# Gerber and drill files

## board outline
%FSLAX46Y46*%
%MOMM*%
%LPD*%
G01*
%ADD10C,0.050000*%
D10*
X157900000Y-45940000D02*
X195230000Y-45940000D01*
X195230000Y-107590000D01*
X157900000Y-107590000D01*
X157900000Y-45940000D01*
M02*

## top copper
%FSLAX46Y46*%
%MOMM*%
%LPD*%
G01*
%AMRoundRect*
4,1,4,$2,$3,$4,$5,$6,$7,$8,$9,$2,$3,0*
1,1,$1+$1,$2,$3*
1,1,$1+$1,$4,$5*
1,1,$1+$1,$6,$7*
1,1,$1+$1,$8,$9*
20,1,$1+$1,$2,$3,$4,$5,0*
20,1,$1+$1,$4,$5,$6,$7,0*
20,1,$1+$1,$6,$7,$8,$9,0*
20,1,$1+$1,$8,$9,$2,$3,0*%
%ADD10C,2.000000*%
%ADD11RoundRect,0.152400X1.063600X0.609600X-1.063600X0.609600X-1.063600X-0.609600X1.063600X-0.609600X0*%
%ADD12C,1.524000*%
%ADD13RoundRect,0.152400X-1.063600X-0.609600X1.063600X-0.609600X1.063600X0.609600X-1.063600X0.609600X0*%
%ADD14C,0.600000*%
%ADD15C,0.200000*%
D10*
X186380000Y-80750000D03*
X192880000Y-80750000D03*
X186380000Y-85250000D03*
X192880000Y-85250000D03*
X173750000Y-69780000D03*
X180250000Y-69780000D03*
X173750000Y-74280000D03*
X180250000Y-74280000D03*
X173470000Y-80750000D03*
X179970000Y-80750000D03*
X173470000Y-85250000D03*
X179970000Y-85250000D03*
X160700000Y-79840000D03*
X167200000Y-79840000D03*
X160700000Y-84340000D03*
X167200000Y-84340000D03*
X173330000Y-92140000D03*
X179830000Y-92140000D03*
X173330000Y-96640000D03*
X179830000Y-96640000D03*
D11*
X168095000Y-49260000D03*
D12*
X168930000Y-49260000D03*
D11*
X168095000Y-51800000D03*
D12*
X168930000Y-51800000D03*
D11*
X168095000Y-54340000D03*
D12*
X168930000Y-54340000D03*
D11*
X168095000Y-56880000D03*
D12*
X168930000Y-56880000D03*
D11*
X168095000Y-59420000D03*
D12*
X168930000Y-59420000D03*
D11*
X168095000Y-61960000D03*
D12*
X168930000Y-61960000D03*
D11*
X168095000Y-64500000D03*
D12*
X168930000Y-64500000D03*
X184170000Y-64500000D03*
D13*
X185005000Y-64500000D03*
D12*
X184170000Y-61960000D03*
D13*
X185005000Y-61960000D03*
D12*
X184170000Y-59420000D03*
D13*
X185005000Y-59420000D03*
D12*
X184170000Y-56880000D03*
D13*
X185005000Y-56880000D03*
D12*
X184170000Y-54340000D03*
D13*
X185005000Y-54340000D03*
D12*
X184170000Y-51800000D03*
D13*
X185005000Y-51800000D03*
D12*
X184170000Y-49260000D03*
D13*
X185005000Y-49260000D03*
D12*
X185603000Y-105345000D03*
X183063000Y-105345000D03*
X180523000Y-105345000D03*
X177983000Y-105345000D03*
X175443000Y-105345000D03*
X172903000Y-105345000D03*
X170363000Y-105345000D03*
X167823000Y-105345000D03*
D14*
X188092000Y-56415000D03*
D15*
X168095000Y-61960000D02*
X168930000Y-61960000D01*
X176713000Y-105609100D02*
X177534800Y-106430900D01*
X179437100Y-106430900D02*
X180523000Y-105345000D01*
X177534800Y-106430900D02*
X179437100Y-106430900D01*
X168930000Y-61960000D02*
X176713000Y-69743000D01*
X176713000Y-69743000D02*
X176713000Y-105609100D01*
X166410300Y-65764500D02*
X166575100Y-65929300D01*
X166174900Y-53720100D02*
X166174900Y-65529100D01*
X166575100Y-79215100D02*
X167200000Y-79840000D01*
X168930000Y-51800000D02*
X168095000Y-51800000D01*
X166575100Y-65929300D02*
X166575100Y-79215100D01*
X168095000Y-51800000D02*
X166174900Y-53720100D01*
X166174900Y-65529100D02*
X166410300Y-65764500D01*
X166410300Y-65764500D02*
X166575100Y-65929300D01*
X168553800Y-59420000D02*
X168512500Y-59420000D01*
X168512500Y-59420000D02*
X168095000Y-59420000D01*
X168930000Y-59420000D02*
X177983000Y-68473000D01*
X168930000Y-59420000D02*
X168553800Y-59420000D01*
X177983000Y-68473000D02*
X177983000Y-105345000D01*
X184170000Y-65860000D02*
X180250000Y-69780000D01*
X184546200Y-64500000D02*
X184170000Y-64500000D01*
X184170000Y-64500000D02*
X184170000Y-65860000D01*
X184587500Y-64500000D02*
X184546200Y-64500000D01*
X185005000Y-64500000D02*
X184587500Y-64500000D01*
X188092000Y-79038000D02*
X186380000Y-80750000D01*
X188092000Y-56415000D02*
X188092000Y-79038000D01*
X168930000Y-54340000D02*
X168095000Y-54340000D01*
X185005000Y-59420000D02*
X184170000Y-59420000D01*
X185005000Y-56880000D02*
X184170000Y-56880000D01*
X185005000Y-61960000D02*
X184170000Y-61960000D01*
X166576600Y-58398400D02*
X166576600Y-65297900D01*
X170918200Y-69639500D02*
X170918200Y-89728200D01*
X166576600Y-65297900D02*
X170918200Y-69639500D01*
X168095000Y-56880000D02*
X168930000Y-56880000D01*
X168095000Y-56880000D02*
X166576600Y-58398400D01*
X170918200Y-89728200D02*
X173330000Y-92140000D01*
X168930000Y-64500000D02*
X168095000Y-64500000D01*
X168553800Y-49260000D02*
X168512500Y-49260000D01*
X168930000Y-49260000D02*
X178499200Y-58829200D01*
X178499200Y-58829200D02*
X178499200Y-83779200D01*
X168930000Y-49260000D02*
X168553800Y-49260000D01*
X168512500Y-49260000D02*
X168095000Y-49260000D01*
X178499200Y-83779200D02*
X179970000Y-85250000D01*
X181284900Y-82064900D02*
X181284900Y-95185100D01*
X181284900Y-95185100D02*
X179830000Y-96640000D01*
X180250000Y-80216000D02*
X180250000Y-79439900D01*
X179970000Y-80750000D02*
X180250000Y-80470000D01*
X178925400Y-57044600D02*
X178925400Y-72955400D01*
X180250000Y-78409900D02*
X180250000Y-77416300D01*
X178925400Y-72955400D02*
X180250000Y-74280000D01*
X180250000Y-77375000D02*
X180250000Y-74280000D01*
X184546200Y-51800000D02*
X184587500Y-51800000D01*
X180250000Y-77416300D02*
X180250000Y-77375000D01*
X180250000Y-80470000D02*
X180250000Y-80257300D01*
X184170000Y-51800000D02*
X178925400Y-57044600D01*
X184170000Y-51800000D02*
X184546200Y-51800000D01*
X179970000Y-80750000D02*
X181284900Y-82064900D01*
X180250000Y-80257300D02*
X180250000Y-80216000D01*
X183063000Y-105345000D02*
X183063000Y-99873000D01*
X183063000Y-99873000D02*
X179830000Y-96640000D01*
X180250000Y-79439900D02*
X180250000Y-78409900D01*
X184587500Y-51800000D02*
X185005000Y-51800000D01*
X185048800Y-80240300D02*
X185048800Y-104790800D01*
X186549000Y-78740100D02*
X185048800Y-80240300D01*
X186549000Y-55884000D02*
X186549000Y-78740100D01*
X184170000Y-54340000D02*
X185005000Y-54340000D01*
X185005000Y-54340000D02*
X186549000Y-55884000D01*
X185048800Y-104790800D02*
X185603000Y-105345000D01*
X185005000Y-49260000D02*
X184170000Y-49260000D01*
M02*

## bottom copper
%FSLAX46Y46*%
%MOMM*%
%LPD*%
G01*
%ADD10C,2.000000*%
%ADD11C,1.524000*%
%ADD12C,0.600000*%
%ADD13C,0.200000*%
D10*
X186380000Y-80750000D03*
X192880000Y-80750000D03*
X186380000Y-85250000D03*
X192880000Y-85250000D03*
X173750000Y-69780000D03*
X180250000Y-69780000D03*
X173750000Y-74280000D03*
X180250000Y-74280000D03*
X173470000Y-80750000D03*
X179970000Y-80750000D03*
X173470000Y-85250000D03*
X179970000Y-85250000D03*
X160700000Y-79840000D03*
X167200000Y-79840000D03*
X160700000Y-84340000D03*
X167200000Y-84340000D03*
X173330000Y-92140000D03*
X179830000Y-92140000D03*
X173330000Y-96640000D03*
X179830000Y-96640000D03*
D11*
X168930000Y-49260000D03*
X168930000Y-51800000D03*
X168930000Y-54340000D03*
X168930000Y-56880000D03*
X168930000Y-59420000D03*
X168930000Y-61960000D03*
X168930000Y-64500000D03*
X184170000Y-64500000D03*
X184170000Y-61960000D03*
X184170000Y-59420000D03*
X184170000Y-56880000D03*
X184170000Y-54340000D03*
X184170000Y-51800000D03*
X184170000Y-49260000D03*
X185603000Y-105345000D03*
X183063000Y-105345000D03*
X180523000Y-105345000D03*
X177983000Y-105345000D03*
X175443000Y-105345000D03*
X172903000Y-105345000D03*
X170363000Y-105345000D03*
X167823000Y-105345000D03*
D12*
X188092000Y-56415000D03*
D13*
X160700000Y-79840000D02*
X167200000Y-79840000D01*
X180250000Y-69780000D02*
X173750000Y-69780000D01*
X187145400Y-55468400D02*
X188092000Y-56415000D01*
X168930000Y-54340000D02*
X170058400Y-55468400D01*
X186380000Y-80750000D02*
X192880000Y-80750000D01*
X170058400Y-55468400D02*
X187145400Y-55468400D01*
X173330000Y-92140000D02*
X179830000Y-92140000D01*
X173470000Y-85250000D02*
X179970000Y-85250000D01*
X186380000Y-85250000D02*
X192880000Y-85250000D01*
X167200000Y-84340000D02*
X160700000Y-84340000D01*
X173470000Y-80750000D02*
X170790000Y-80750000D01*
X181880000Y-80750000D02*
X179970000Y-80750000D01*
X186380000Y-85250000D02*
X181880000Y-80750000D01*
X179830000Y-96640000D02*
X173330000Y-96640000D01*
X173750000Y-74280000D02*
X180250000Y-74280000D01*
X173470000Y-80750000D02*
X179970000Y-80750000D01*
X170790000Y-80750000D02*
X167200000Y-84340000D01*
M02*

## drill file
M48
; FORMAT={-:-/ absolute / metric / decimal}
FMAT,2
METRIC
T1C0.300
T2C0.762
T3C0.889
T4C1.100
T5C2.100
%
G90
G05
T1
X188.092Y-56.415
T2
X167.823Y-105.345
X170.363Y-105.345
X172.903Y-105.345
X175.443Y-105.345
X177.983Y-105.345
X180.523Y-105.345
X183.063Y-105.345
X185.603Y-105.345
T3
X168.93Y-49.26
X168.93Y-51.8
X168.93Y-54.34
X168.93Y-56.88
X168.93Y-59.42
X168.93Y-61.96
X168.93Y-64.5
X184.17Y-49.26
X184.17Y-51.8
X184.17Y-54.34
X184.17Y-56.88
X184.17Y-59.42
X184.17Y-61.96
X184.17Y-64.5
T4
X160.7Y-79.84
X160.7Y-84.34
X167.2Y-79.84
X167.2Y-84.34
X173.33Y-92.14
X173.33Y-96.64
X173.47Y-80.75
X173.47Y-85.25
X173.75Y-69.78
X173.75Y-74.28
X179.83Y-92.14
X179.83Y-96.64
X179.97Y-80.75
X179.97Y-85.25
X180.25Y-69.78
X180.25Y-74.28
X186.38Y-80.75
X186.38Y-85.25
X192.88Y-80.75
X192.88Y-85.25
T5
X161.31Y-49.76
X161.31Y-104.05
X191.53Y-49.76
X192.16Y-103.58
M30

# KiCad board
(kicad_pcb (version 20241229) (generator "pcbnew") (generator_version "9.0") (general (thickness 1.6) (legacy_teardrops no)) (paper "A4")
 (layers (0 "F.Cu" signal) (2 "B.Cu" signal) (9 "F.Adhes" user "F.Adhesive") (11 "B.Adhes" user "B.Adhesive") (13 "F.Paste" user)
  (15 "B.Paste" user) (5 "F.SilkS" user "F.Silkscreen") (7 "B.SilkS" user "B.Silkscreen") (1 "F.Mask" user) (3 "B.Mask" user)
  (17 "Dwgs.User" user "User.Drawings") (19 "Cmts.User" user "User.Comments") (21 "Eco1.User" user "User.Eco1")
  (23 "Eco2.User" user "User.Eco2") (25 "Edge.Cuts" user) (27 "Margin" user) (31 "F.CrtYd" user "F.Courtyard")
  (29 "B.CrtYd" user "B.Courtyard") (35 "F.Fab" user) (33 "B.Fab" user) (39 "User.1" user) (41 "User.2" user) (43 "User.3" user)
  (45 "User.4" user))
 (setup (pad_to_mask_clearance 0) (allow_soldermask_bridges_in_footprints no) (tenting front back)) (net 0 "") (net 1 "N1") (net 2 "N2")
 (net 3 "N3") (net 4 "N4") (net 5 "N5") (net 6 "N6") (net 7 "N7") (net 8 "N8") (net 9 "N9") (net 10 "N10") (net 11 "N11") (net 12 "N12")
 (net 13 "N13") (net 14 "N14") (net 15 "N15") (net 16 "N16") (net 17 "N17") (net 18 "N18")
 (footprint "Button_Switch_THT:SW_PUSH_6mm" (layer "F.Cu") (at 186.38 80.75)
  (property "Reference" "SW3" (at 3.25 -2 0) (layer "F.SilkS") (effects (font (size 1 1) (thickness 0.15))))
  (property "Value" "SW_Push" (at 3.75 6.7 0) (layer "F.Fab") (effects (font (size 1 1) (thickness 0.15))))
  (pad "1" thru_hole circle (at 0 0 90) (size 2 2) (drill 1.1) (layers "*.Cu" "*.Mask") (remove_unused_layers no) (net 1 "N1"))
  (pad "1" thru_hole circle (at 6.5 0 90) (size 2 2) (drill 1.1) (layers "*.Cu" "*.Mask") (remove_unused_layers no) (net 1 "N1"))
  (pad "2" thru_hole circle (at 0 4.5 90) (size 2 2) (drill 1.1) (layers "*.Cu" "*.Mask") (remove_unused_layers no) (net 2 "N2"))
  (pad "2" thru_hole circle (at 6.5 4.5 90) (size 2 2) (drill 1.1) (layers "*.Cu" "*.Mask") (remove_unused_layers no) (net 2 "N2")))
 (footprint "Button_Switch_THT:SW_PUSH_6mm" (layer "F.Cu") (at 173.75 69.78)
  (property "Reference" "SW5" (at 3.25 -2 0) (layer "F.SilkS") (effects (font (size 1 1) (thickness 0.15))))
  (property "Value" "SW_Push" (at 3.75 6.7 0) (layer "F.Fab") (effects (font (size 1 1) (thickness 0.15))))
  (pad "1" thru_hole circle (at 0 0 90) (size 2 2) (drill 1.1) (layers "*.Cu" "*.Mask") (remove_unused_layers no) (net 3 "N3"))
  (pad "1" thru_hole circle (at 6.5 0 90) (size 2 2) (drill 1.1) (layers "*.Cu" "*.Mask") (remove_unused_layers no) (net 3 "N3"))
  (pad "2" thru_hole circle (at 0 4.5 90) (size 2 2) (drill 1.1) (layers "*.Cu" "*.Mask") (remove_unused_layers no) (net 2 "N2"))
  (pad "2" thru_hole circle (at 6.5 4.5 90) (size 2 2) (drill 1.1) (layers "*.Cu" "*.Mask") (remove_unused_layers no) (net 2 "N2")))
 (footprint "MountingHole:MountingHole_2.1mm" (layer "F.Cu") (at 192.16 103.58)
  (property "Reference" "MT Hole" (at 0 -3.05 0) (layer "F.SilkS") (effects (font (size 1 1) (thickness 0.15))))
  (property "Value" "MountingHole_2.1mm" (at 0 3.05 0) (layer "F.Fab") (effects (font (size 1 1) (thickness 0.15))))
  (pad "" np_thru_hole circle (at 0 0) (size 2.1 2.1) (drill 2.1) (layers "*.Cu" "*.Mask")))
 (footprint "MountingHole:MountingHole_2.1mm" (layer "F.Cu") (at 161.31 49.76)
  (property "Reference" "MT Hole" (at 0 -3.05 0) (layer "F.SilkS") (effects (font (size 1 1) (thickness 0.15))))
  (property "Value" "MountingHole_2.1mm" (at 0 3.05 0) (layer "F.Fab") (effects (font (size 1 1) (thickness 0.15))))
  (pad "" np_thru_hole circle (at 0 0) (size 2.1 2.1) (drill 2.1) (layers "*.Cu" "*.Mask")))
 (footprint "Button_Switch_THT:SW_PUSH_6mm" (layer "F.Cu") (at 173.47 80.75)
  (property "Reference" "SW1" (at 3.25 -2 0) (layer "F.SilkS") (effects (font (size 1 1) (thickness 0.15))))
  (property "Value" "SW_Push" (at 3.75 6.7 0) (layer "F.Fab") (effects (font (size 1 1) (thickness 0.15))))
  (pad "1" thru_hole circle (at 0 0 90) (size 2 2) (drill 1.1) (layers "*.Cu" "*.Mask") (remove_unused_layers no) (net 2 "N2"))
  (pad "1" thru_hole circle (at 6.5 0 90) (size 2 2) (drill 1.1) (layers "*.Cu" "*.Mask") (remove_unused_layers no) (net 2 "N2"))
  (pad "2" thru_hole circle (at 0 4.5 90) (size 2 2) (drill 1.1) (layers "*.Cu" "*.Mask") (remove_unused_layers no) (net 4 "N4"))
  (pad "2" thru_hole circle (at 6.5 4.5 90) (size 2 2) (drill 1.1) (layers "*.Cu" "*.Mask") (remove_unused_layers no) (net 4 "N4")))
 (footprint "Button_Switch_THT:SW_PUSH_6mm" (layer "F.Cu") (at 160.7 79.84)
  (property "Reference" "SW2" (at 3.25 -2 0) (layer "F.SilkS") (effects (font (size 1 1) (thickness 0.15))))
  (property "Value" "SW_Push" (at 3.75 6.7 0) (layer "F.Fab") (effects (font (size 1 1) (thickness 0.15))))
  (pad "1" thru_hole circle (at 0 0 90) (size 2 2) (drill 1.1) (layers "*.Cu" "*.Mask") (remove_unused_layers no) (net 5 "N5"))
  (pad "1" thru_hole circle (at 6.5 0 90) (size 2 2) (drill 1.1) (layers "*.Cu" "*.Mask") (remove_unused_layers no) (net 5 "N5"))
  (pad "2" thru_hole circle (at 0 4.5 90) (size 2 2) (drill 1.1) (layers "*.Cu" "*.Mask") (remove_unused_layers no) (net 2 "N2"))
  (pad "2" thru_hole circle (at 6.5 4.5 90) (size 2 2) (drill 1.1) (layers "*.Cu" "*.Mask") (remove_unused_layers no) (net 2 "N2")))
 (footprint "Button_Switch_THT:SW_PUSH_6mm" (layer "F.Cu") (at 173.33 92.14)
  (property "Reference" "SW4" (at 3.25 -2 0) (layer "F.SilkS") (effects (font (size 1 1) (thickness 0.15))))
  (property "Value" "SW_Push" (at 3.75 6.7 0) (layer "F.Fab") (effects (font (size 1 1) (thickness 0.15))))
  (pad "1" thru_hole circle (at 0 0 90) (size 2 2) (drill 1.1) (layers "*.Cu" "*.Mask") (remove_unused_layers no) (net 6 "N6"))
  (pad "1" thru_hole circle (at 6.5 0 90) (size 2 2) (drill 1.1) (layers "*.Cu" "*.Mask") (remove_unused_layers no) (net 6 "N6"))
  (pad "2" thru_hole circle (at 0 4.5 90) (size 2 2) (drill 1.1) (layers "*.Cu" "*.Mask") (remove_unused_layers no) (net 2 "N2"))
  (pad "2" thru_hole circle (at 6.5 4.5 90) (size 2 2) (drill 1.1) (layers "*.Cu" "*.Mask") (remove_unused_layers no) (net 2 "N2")))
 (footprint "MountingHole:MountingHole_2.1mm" (layer "F.Cu") (at 191.53 49.76)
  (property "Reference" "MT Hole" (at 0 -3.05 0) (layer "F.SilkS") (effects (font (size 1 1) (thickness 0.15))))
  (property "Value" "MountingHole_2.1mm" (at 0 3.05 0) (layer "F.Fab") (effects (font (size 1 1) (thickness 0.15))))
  (pad "" np_thru_hole circle (at 0 0) (size 2.1 2.1) (drill 2.1) (layers "*.Cu" "*.Mask")))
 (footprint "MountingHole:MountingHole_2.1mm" (layer "F.Cu") (at 161.31 104.05)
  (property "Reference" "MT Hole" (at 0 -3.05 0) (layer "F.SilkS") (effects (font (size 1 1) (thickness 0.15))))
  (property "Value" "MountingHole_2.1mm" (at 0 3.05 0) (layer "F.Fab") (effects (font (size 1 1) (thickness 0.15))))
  (pad "" np_thru_hole circle (at 0 0) (size 2.1 2.1) (drill 2.1) (layers "*.Cu" "*.Mask")))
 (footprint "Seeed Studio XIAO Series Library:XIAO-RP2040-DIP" (layer "F.Cu") (at 176.55 56.88)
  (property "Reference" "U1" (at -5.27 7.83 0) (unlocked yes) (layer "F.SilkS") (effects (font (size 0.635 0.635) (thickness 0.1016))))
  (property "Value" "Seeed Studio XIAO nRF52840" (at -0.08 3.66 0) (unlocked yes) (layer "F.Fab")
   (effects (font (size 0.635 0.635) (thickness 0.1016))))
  (pad "1" smd roundrect (at -8.455 -7.62 180) (size 2.432 1.524) (layers "F.Cu" "F.Mask") (roundrect_rratio 0.1) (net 4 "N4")
   (thermal_bridge_angle 45))
  (pad "1" thru_hole circle (at -7.62 -7.62 180) (size 1.524 1.524) (drill 0.889) (layers "*.Cu" "*.Mask") (remove_unused_layers no)
   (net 4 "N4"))
  (pad "2" smd roundrect (at -8.455 -5.08 180) (size 2.432 1.524) (layers "F.Cu" "F.Mask") (roundrect_rratio 0.1) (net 5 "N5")
   (thermal_bridge_angle 45))
  (pad "2" thru_hole circle (at -7.62 -5.08 180) (size 1.524 1.524) (drill 0.889) (layers "*.Cu" "*.Mask") (remove_unused_layers no)
   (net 5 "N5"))
  (pad "3" smd roundrect (at -8.455 -2.54 180) (size 2.432 1.524) (layers "F.Cu" "F.Mask") (roundrect_rratio 0.1) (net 1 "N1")
   (thermal_bridge_angle 45))
  (pad "3" thru_hole circle (at -7.62 -2.54 180) (size 1.524 1.524) (drill 0.889) (layers "*.Cu" "*.Mask") (remove_unused_layers no)
   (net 1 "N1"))
  (pad "4" smd roundrect (at -8.455 0 180) (size 2.432 1.524) (layers "F.Cu" "F.Mask") (roundrect_rratio 0.1) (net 6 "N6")
   (thermal_bridge_angle 45))
  (pad "4" thru_hole circle (at -7.62 0 180) (size 1.524 1.524) (drill 0.889) (layers "*.Cu" "*.Mask") (remove_unused_layers no)
   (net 6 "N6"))
  (pad "5" smd roundrect (at -8.455 2.54 180) (size 2.432 1.524) (layers "F.Cu" "F.Mask") (roundrect_rratio 0.1) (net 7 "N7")
   (thermal_bridge_angle 45))
  (pad "5" thru_hole circle (at -7.62 2.54 180) (size 1.524 1.524) (drill 0.889) (layers "*.Cu" "*.Mask") (remove_unused_layers no)
   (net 7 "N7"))
  (pad "6" smd roundrect (at -8.455 5.08 180) (size 2.432 1.524) (layers "F.Cu" "F.Mask") (roundrect_rratio 0.1) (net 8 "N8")
   (thermal_bridge_angle 45))
  (pad "6" thru_hole circle (at -7.62 5.08 180) (size 1.524 1.524) (drill 0.889) (layers "*.Cu" "*.Mask") (remove_unused_layers no)
   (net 8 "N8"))
  (pad "7" smd roundrect (at -8.455 7.62 180) (size 2.432 1.524) (layers "F.Cu" "F.Mask") (roundrect_rratio 0.1) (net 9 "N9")
   (thermal_bridge_angle 45))
  (pad "7" thru_hole circle (at -7.62 7.62 180) (size 1.524 1.524) (drill 0.889) (layers "*.Cu" "*.Mask") (remove_unused_layers no)
   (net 9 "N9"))
  (pad "8" thru_hole circle (at 7.62 7.62) (size 1.524 1.524) (drill 0.889) (layers "*.Cu" "*.Mask") (remove_unused_layers no) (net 3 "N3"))
  (pad "8" smd roundrect (at 8.455 7.62) (size 2.432 1.524) (layers "F.Cu" "F.Mask") (roundrect_rratio 0.1) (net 3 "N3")
   (thermal_bridge_angle 45))
  (pad "9" thru_hole circle (at 7.62 5.08) (size 1.524 1.524) (drill 0.889) (layers "*.Cu" "*.Mask") (remove_unused_layers no)
   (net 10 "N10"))
  (pad "9" smd roundrect (at 8.455 5.08) (size 2.432 1.524) (layers "F.Cu" "F.Mask") (roundrect_rratio 0.1) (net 10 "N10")
   (thermal_bridge_angle 45))
  (pad "10" thru_hole circle (at 7.62 2.54) (size 1.524 1.524) (drill 0.889) (layers "*.Cu" "*.Mask") (remove_unused_layers no)
   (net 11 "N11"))
  (pad "10" smd roundrect (at 8.455 2.54) (size 2.432 1.524) (layers "F.Cu" "F.Mask") (roundrect_rratio 0.1) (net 11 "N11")
   (thermal_bridge_angle 45))
  (pad "11" thru_hole circle (at 7.62 0) (size 1.524 1.524) (drill 0.889) (layers "*.Cu" "*.Mask") (remove_unused_layers no) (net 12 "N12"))
  (pad "11" smd roundrect (at 8.455 0) (size 2.432 1.524) (layers "F.Cu" "F.Mask") (roundrect_rratio 0.1) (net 12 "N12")
   (thermal_bridge_angle 45))
  (pad "12" thru_hole circle (at 7.62 -2.54) (size 1.524 1.524) (drill 0.889) (layers "*.Cu" "*.Mask") (remove_unused_layers no)
   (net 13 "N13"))
  (pad "12" smd roundrect (at 8.455 -2.54) (size 2.432 1.524) (layers "F.Cu" "F.Mask") (roundrect_rratio 0.1) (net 13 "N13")
   (thermal_bridge_angle 45))
  (pad "13" thru_hole circle (at 7.62 -5.08) (size 1.524 1.524) (drill 0.889) (layers "*.Cu" "*.Mask") (remove_unused_layers no)
   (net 2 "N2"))
  (pad "13" smd roundrect (at 8.455 -5.08) (size 2.432 1.524) (layers "F.Cu" "F.Mask") (roundrect_rratio 0.1) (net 2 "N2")
   (thermal_bridge_angle 45))
  (pad "14" thru_hole circle (at 7.62 -7.62) (size 1.524 1.524) (drill 0.889) (layers "*.Cu" "*.Mask") (remove_unused_layers no)
   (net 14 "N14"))
  (pad "14" smd roundrect (at 8.455 -7.62) (size 2.432 1.524) (layers "F.Cu" "F.Mask") (roundrect_rratio 0.1) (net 14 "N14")
   (thermal_bridge_angle 45)))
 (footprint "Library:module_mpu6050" (layer "B.Cu") (at 167.823 105.345 90)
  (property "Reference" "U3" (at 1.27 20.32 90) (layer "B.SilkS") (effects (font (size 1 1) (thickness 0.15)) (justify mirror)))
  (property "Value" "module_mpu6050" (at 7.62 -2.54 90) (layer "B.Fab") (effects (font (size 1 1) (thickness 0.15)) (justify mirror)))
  (pad "1" thru_hole circle (at 0 17.78 90) (size 1.524 1.524) (drill 0.762) (layers "*.Cu" "*.Mask") (remove_unused_layers no)
   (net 13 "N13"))
  (pad "2" thru_hole circle (at 0 15.24 90) (size 1.524 1.524) (drill 0.762) (layers "*.Cu" "*.Mask") (remove_unused_layers no) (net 2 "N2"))
  (pad "3" thru_hole circle (at 0 12.7 90) (size 1.524 1.524) (drill 0.762) (layers "*.Cu" "*.Mask") (remove_unused_layers no) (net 8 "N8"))
  (pad "4" thru_hole circle (at 0 10.16 90) (size 1.524 1.524) (drill 0.762) (layers "*.Cu" "*.Mask") (remove_unused_layers no) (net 7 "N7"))
  (pad "5" thru_hole circle (at 0 7.62 90) (size 1.524 1.524) (drill 0.762) (layers "*.Cu" "*.Mask") (remove_unused_layers no)
   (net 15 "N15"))
  (pad "6" thru_hole circle (at 0 5.08 90) (size 1.524 1.524) (drill 0.762) (layers "*.Cu" "*.Mask") (remove_unused_layers no)
   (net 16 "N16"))
  (pad "7" thru_hole circle (at 0 2.54 90) (size 1.524 1.524) (drill 0.762) (layers "*.Cu" "*.Mask") (remove_unused_layers no)
   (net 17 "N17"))
  (pad "8" thru_hole circle (at 0 0 90) (size 1.524 1.524) (drill 0.762) (layers "*.Cu" "*.Mask") (remove_unused_layers no) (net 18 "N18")))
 (gr_rect (start 157.9 45.94) (end 195.23 107.59) (stroke (width 0.05) (type default)) (fill no) (layer "Edge.Cuts"))
 (segment (start 168.095 61.96) (end 168.93 61.96) (width 0.2) (layer "F.Cu") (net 8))
 (segment (start 176.713 105.6091) (end 177.5348 106.4309) (width 0.2) (layer "F.Cu") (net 8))
 (segment (start 179.4371 106.4309) (end 180.523 105.345) (width 0.2) (layer "F.Cu") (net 8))
 (segment (start 177.5348 106.4309) (end 179.4371 106.4309) (width 0.2) (layer "F.Cu") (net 8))
 (segment (start 168.93 61.96) (end 176.713 69.743) (width 0.2) (layer "F.Cu") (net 8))
 (segment (start 176.713 69.743) (end 176.713 105.6091) (width 0.2) (layer "F.Cu") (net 8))
 (segment (start 166.4103 65.7645) (end 166.5751 65.9293) (width 0.2) (layer "F.Cu") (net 5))
 (segment (start 166.1749 53.7201) (end 166.1749 65.5291) (width 0.2) (layer "F.Cu") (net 5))
 (segment (start 166.5751 79.2151) (end 167.2 79.84) (width 0.2) (layer "F.Cu") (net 5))
 (segment (start 168.93 51.8) (end 168.095 51.8) (width 0.2) (layer "F.Cu") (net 5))
 (segment (start 166.5751 65.9293) (end 166.5751 79.2151) (width 0.2) (layer "F.Cu") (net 5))
 (segment (start 168.095 51.8) (end 166.1749 53.7201) (width 0.2) (layer "F.Cu") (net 5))
 (segment (start 166.1749 65.5291) (end 166.4103 65.7645) (width 0.2) (layer "F.Cu") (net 5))
 (segment (start 166.4103 65.7645) (end 166.5751 65.9293) (width 0.2) (layer "F.Cu") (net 5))
 (segment (start 160.7 79.84) (end 167.2 79.84) (width 0.2) (layer "B.Cu") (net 5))
 (segment (start 168.5538 59.42) (end 168.5125 59.42) (width 0.2) (layer "F.Cu") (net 7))
 (segment (start 168.5125 59.42) (end 168.095 59.42) (width 0.2) (layer "F.Cu") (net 7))
 (segment (start 168.93 59.42) (end 177.983 68.473) (width 0.2) (layer "F.Cu") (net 7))
 (segment (start 168.93 59.42) (end 168.5538 59.42) (width 0.2) (layer "F.Cu") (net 7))
 (segment (start 177.983 68.473) (end 177.983 105.345) (width 0.2) (layer "F.Cu") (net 7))
 (segment (start 184.17 65.86) (end 180.25 69.78) (width 0.2) (layer "F.Cu") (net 3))
 (segment (start 184.5462 64.5) (end 184.17 64.5) (width 0.2) (layer "F.Cu") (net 3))
 (segment (start 184.17 64.5) (end 184.17 65.86) (width 0.2) (layer "F.Cu") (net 3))
 (segment (start 184.5875 64.5) (end 184.5462 64.5) (width 0.2) (layer "F.Cu") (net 3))
 (segment (start 185.005 64.5) (end 184.5875 64.5) (width 0.2) (layer "F.Cu") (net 3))
 (segment (start 180.25 69.78) (end 173.75 69.78) (width 0.2) (layer "B.Cu") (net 3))
 (segment (start 188.092 79.038) (end 186.38 80.75) (width 0.2) (layer "F.Cu") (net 1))
 (segment (start 188.092 56.415) (end 188.092 79.038) (width 0.2) (layer "F.Cu") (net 1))
 (segment (start 168.93 54.34) (end 168.095 54.34) (width 0.2) (layer "F.Cu") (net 1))
 (via (at 188.092 56.415) (size 0.6) (drill 0.3) (layers "F.Cu" "B.Cu") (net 1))
 (segment (start 187.1454 55.4684) (end 188.092 56.415) (width 0.2) (layer "B.Cu") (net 1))
 (segment (start 168.93 54.34) (end 170.0584 55.4684) (width 0.2) (layer "B.Cu") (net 1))
 (segment (start 186.38 80.75) (end 192.88 80.75) (width 0.2) (layer "B.Cu") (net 1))
 (segment (start 170.0584 55.4684) (end 187.1454 55.4684) (width 0.2) (layer "B.Cu") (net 1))
 (segment (start 185.005 59.42) (end 184.17 59.42) (width 0.2) (layer "F.Cu") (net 11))
 (segment (start 185.005 56.88) (end 184.17 56.88) (width 0.2) (layer "F.Cu") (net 12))
 (segment (start 185.005 61.96) (end 184.17 61.96) (width 0.2) (layer "F.Cu") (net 10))
 (segment (start 166.5766 58.3984) (end 166.5766 65.2979) (width 0.2) (layer "F.Cu") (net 6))
 (segment (start 170.9182 69.6395) (end 170.9182 89.7282) (width 0.2) (layer "F.Cu") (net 6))
 (segment (start 166.5766 65.2979) (end 170.9182 69.6395) (width 0.2) (layer "F.Cu") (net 6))
 (segment (start 168.095 56.88) (end 168.93 56.88) (width 0.2) (layer "F.Cu") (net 6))
 (segment (start 168.095 56.88) (end 166.5766 58.3984) (width 0.2) (layer "F.Cu") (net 6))
 (segment (start 170.9182 89.7282) (end 173.33 92.14) (width 0.2) (layer "F.Cu") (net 6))
 (segment (start 173.33 92.14) (end 179.83 92.14) (width 0.2) (layer "B.Cu") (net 6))
 (segment (start 168.93 64.5) (end 168.095 64.5) (width 0.2) (layer "F.Cu") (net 9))
 (segment (start 168.5538 49.26) (end 168.5125 49.26) (width 0.2) (layer "F.Cu") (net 4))
 (segment (start 168.93 49.26) (end 178.4992 58.8292) (width 0.2) (layer "F.Cu") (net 4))
 (segment (start 178.4992 58.8292) (end 178.4992 83.7792) (width 0.2) (layer "F.Cu") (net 4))
 (segment (start 168.93 49.26) (end 168.5538 49.26) (width 0.2) (layer "F.Cu") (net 4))
 (segment (start 168.5125 49.26) (end 168.095 49.26) (width 0.2) (layer "F.Cu") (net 4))
 (segment (start 178.4992 83.7792) (end 179.97 85.25) (width 0.2) (layer "F.Cu") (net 4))
 (segment (start 173.47 85.25) (end 179.97 85.25) (width 0.2) (layer "B.Cu") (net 4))
 (segment (start 181.2849 82.0649) (end 181.2849 95.1851) (width 0.2) (layer "F.Cu") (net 2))
 (segment (start 181.2849 95.1851) (end 179.83 96.64) (width 0.2) (layer "F.Cu") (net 2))
 (segment (start 180.25 80.216) (end 180.25 79.4399) (width 0.2) (layer "F.Cu") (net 2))
 (segment (start 179.97 80.75) (end 180.25 80.47) (width 0.2) (layer "F.Cu") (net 2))
 (segment (start 178.9254 57.0446) (end 178.9254 72.9554) (width 0.2) (layer "F.Cu") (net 2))
 (segment (start 180.25 78.4099) (end 180.25 77.4163) (width 0.2) (layer "F.Cu") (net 2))
 (segment (start 178.9254 72.9554) (end 180.25 74.28) (width 0.2) (layer "F.Cu") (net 2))
 (segment (start 180.25 77.375) (end 180.25 74.28) (width 0.2) (layer "F.Cu") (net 2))
 (segment (start 184.5462 51.8) (end 184.5875 51.8) (width 0.2) (layer "F.Cu") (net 2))
 (segment (start 180.25 77.4163) (end 180.25 77.375) (width 0.2) (layer "F.Cu") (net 2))
 (segment (start 180.25 80.47) (end 180.25 80.2573) (width 0.2) (layer "F.Cu") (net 2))
 (segment (start 184.17 51.8) (end 178.9254 57.0446) (width 0.2) (layer "F.Cu") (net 2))
 (segment (start 184.17 51.8) (end 184.5462 51.8) (width 0.2) (layer "F.Cu") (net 2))
 (segment (start 179.97 80.75) (end 181.2849 82.0649) (width 0.2) (layer "F.Cu") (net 2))
 (segment (start 180.25 80.2573) (end 180.25 80.216) (width 0.2) (layer "F.Cu") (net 2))
 (segment (start 183.063 105.345) (end 183.063 99.873) (width 0.2) (layer "F.Cu") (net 2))
 (segment (start 183.063 99.873) (end 179.83 96.64) (width 0.2) (layer "F.Cu") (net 2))
 (segment (start 180.25 79.4399) (end 180.25 78.4099) (width 0.2) (layer "F.Cu") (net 2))
 (segment (start 184.5875 51.8) (end 185.005 51.8) (width 0.2) (layer "F.Cu") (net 2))
 (segment (start 186.38 85.25) (end 192.88 85.25) (width 0.2) (layer "B.Cu") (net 2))
 (segment (start 167.2 84.34) (end 160.7 84.34) (width 0.2) (layer "B.Cu") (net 2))
 (segment (start 173.47 80.75) (end 170.79 80.75) (width 0.2) (layer "B.Cu") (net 2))
 (segment (start 181.88 80.75) (end 179.97 80.75) (width 0.2) (layer "B.Cu") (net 2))
 (segment (start 186.38 85.25) (end 181.88 80.75) (width 0.2) (layer "B.Cu") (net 2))
 (segment (start 179.83 96.64) (end 173.33 96.64) (width 0.2) (layer "B.Cu") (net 2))
 (segment (start 173.75 74.28) (end 180.25 74.28) (width 0.2) (layer "B.Cu") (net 2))
 (segment (start 173.47 80.75) (end 179.97 80.75) (width 0.2) (layer "B.Cu") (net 2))
 (segment (start 170.79 80.75) (end 167.2 84.34) (width 0.2) (layer "B.Cu") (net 2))
 (segment (start 185.0488 80.2403) (end 185.0488 104.7908) (width 0.2) (layer "F.Cu") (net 13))
 (segment (start 186.549 78.7401) (end 185.0488 80.2403) (width 0.2) (layer "F.Cu") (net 13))
 (segment (start 186.549 55.884) (end 186.549 78.7401) (width 0.2) (layer "F.Cu") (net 13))
 (segment (start 184.17 54.34) (end 185.005 54.34) (width 0.2) (layer "F.Cu") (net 13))
 (segment (start 185.005 54.34) (end 186.549 55.884) (width 0.2) (layer "F.Cu") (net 13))
 (segment (start 185.0488 104.7908) (end 185.603 105.345) (width 0.2) (layer "F.Cu") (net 13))
 (segment (start 185.005 49.26) (end 184.17 49.26) (width 0.2) (layer "F.Cu") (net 14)))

